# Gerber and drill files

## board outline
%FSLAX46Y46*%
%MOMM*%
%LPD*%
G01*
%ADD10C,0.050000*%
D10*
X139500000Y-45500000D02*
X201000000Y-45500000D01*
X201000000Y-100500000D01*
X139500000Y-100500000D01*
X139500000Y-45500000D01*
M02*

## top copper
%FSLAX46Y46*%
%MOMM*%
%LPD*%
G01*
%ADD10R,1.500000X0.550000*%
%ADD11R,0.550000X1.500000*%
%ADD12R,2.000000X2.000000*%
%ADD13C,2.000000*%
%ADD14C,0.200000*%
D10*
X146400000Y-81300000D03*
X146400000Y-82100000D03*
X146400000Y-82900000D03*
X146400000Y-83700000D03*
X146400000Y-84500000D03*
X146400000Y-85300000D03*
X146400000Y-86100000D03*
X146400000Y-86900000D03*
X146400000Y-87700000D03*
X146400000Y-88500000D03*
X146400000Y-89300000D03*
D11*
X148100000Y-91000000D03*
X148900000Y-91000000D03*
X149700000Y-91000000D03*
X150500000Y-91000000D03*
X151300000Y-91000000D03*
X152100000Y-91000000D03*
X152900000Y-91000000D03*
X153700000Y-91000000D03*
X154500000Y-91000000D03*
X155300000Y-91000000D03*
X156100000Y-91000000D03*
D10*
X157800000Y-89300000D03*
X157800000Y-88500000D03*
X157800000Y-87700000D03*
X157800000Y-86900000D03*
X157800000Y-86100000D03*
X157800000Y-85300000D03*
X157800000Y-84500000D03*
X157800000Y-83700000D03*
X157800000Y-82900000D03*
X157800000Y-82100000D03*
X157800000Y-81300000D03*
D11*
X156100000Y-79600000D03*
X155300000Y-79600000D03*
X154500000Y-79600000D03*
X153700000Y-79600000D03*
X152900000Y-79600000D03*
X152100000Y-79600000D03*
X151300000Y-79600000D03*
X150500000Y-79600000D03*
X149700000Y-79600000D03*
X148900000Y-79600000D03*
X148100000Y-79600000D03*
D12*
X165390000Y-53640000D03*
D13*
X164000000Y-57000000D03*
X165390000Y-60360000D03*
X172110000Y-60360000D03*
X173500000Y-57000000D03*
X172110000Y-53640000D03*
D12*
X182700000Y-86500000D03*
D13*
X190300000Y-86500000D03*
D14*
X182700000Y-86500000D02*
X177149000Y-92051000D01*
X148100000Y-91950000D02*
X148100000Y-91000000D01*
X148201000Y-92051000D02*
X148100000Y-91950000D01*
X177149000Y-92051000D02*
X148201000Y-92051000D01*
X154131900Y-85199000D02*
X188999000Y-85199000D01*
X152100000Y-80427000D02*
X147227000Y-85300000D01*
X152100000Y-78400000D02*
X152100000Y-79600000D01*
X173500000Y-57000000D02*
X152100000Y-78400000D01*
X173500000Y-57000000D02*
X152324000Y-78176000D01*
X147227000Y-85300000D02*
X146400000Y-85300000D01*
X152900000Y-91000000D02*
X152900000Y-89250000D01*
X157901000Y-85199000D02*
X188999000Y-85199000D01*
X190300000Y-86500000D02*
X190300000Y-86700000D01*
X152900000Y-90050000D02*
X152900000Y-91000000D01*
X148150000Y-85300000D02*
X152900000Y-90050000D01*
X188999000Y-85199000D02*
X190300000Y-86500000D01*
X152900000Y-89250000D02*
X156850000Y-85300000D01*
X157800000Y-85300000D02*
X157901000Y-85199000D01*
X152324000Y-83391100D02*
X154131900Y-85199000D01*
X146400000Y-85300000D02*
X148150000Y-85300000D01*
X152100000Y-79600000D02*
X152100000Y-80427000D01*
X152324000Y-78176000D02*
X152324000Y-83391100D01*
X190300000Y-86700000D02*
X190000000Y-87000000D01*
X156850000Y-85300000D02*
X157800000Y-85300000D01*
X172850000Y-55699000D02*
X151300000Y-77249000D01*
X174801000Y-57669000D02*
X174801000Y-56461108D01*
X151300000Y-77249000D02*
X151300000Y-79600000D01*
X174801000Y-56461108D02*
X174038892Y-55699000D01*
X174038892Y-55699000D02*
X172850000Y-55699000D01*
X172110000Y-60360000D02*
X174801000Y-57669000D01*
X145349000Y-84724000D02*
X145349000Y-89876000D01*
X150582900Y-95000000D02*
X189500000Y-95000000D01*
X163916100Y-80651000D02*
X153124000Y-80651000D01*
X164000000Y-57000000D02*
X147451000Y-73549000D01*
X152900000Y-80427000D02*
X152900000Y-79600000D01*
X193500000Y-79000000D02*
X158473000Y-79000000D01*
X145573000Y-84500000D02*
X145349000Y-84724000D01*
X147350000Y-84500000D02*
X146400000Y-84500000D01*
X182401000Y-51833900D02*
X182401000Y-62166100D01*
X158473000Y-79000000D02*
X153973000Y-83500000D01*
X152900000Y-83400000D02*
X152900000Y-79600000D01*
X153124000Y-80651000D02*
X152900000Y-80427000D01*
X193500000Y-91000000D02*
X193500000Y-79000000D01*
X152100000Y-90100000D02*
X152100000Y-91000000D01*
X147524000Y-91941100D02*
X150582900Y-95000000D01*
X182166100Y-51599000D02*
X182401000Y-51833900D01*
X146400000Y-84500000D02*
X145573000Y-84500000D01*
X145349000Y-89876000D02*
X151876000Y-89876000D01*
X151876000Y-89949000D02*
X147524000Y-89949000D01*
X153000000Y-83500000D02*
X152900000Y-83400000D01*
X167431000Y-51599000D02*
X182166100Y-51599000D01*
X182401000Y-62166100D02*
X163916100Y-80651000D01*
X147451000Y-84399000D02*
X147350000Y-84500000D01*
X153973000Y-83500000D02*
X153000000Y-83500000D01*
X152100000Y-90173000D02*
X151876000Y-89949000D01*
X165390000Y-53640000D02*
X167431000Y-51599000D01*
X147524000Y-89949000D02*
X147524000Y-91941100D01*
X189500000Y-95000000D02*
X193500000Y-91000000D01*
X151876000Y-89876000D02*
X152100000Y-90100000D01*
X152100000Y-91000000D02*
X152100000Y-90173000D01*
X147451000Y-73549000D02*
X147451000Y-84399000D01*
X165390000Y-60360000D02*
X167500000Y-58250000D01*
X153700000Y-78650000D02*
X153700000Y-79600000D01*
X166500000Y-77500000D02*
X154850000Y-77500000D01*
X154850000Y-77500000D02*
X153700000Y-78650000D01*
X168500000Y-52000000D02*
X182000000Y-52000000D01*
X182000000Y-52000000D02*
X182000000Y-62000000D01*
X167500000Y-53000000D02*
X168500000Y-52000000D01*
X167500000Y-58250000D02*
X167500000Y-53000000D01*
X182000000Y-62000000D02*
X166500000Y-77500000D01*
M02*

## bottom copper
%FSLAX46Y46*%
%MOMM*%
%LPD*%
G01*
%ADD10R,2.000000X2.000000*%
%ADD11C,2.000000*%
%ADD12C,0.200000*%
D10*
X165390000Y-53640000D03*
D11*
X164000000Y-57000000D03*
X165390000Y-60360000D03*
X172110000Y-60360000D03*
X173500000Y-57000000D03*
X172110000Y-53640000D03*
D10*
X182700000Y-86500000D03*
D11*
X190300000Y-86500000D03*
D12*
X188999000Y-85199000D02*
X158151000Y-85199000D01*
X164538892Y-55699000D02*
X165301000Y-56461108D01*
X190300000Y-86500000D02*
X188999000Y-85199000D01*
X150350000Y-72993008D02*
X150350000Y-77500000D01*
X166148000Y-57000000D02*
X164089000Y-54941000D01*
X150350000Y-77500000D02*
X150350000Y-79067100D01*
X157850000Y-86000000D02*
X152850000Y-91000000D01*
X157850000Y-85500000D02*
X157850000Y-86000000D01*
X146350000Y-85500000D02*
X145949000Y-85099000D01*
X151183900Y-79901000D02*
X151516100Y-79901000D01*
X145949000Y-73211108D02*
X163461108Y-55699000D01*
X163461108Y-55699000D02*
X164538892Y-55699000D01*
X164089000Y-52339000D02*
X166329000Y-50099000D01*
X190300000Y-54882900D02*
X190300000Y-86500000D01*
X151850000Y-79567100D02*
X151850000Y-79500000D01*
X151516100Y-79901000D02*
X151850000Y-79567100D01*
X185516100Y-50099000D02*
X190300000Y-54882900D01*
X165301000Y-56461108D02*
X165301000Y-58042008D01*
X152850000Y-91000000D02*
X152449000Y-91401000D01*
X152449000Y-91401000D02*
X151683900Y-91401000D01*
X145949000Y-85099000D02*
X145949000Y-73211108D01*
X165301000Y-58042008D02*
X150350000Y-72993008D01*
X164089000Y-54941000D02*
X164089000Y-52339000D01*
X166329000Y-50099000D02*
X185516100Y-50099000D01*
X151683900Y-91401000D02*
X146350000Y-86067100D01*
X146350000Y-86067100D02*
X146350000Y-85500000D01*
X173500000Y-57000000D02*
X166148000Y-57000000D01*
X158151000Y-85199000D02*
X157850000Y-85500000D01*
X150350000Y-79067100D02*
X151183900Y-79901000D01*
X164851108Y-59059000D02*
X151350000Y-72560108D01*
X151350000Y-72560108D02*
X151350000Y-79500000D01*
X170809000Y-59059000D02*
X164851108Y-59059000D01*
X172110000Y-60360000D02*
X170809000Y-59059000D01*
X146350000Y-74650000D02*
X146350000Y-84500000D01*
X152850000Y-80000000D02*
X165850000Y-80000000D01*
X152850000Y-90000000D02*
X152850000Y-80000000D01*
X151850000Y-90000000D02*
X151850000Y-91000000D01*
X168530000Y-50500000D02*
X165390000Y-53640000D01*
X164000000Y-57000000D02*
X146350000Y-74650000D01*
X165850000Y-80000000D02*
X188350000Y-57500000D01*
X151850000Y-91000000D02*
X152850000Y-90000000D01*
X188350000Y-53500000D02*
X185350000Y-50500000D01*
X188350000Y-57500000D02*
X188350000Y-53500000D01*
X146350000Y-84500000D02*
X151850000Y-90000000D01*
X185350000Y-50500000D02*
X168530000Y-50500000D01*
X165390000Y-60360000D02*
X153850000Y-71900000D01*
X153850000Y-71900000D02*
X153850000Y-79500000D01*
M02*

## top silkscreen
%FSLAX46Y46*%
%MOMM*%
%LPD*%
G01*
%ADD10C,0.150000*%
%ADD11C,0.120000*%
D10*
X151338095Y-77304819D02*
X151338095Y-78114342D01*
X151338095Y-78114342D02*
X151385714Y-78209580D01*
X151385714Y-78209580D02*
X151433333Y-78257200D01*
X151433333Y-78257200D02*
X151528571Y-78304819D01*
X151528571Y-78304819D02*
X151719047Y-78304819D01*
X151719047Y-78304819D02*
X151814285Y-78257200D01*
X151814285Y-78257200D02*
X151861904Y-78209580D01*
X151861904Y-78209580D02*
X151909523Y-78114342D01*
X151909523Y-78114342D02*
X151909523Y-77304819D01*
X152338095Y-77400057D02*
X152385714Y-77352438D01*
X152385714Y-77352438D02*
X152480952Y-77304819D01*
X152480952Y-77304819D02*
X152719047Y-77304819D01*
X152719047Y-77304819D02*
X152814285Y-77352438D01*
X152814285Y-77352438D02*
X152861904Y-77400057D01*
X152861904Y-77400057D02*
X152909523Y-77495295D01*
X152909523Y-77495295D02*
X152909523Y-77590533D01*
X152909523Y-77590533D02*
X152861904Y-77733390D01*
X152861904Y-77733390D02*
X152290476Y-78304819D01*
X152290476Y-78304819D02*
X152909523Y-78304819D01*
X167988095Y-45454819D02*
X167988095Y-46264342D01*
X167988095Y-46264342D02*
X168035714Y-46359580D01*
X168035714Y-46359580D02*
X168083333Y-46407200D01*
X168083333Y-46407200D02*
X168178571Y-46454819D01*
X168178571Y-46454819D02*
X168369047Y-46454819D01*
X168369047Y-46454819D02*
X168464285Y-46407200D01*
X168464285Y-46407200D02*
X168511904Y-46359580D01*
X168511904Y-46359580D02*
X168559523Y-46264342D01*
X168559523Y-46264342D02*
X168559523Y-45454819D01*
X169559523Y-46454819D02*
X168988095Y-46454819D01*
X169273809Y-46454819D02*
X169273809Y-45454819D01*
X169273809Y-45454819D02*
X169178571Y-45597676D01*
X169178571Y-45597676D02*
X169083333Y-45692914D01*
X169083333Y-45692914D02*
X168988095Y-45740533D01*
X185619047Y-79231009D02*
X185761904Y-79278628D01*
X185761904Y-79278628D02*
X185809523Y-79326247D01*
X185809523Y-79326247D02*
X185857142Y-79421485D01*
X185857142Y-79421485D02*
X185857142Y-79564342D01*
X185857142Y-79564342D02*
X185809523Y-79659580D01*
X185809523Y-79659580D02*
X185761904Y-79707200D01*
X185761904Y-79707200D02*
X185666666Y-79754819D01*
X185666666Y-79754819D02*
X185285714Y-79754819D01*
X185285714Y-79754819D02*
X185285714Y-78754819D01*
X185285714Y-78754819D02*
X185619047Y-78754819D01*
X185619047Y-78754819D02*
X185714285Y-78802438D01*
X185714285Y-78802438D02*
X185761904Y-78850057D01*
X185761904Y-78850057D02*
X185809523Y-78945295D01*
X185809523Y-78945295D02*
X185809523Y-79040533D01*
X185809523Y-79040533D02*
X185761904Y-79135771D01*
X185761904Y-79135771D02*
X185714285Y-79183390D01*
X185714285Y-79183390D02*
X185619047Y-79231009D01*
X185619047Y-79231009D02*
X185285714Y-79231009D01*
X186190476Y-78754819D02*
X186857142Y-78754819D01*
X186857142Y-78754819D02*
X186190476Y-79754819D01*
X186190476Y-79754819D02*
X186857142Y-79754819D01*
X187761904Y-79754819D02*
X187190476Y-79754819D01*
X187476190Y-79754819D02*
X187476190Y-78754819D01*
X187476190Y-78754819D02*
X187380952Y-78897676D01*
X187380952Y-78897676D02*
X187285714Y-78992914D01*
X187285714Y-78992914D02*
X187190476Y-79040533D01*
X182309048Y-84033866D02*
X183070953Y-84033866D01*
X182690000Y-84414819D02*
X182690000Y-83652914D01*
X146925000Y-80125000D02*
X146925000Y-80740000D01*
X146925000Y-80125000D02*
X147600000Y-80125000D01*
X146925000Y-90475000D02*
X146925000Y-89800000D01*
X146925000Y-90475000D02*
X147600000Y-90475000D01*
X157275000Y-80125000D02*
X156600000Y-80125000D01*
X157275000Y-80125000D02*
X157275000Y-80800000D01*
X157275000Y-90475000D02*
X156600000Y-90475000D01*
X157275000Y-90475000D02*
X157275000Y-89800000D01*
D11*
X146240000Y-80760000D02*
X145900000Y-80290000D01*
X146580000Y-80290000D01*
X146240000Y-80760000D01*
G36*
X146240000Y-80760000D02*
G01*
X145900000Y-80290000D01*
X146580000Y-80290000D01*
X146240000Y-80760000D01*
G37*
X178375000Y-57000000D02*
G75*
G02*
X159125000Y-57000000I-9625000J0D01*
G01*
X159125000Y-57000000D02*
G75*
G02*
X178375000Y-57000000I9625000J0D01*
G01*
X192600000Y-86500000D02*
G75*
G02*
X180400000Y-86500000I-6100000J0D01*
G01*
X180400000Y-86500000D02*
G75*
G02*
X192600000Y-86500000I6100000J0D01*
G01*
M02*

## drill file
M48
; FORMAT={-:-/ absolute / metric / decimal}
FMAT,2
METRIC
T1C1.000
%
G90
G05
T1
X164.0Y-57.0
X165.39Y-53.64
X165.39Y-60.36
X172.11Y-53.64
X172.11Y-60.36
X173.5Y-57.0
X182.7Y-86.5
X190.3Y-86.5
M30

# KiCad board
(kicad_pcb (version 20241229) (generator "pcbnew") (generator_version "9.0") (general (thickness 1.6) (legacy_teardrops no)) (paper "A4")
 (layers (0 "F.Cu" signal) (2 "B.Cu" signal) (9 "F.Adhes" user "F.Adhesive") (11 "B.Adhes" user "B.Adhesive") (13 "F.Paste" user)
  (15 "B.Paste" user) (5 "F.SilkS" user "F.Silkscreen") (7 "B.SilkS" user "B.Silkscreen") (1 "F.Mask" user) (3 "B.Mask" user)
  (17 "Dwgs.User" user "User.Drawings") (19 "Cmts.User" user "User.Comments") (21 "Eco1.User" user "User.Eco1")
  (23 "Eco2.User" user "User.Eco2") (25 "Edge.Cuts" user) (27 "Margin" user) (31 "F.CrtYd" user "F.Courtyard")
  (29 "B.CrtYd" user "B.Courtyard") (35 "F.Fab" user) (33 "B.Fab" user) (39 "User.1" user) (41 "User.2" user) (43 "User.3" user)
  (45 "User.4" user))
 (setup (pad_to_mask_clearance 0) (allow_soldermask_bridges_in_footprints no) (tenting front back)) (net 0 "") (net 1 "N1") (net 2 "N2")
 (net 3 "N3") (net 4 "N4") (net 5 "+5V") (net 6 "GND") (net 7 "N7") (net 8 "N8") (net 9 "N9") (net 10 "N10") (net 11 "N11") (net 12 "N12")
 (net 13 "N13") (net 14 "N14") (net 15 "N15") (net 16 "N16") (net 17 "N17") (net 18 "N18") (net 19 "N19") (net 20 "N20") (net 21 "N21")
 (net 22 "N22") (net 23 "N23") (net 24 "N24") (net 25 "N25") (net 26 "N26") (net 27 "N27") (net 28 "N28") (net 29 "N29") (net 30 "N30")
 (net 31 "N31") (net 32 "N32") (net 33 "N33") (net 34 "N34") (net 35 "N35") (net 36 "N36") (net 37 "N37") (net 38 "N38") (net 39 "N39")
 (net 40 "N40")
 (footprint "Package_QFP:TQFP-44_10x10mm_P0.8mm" (layer "F.Cu") (at 152.1 85.3)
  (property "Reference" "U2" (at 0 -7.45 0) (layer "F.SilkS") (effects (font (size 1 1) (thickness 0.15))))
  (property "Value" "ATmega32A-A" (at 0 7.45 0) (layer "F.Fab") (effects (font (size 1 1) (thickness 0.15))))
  (fp_line (start -5.175 -5.175) (end -5.175 -4.56) (stroke (width 0.15) (type solid)) (layer "F.SilkS"))
  (fp_line (start -5.175 -5.175) (end -4.5 -5.175) (stroke (width 0.15) (type solid)) (layer "F.SilkS"))
  (fp_line (start -5.175 5.175) (end -5.175 4.5) (stroke (width 0.15) (type solid)) (layer "F.SilkS"))
  (fp_line (start -5.175 5.175) (end -4.5 5.175) (stroke (width 0.15) (type solid)) (layer "F.SilkS"))
  (fp_line (start 5.175 -5.175) (end 4.5 -5.175) (stroke (width 0.15) (type solid)) (layer "F.SilkS"))
  (fp_line (start 5.175 -5.175) (end 5.175 -4.5) (stroke (width 0.15) (type solid)) (layer "F.SilkS"))
  (fp_line (start 5.175 5.175) (end 4.5 5.175) (stroke (width 0.15) (type solid)) (layer "F.SilkS"))
  (fp_line (start 5.175 5.175) (end 5.175 4.5) (stroke (width 0.15) (type solid)) (layer "F.SilkS"))
  (fp_poly
   (pts (xy -5.86 -4.54) (xy -6.2 -5.01) (xy -5.52 -5.01) (xy -5.86 -4.54)) (stroke (width 0.12) (type solid)) (fill yes) (layer "F.SilkS"))
  (pad "1" smd rect (at -5.7 -4) (size 1.5 0.55) (layers "F.Cu" "F.Mask" "F.Paste") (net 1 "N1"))
  (pad "2" smd rect (at -5.7 -3.2) (size 1.5 0.55) (layers "F.Cu" "F.Mask" "F.Paste") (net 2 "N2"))
  (pad "3" smd rect (at -5.7 -2.4) (size 1.5 0.55) (layers "F.Cu" "F.Mask" "F.Paste") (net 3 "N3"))
  (pad "4" smd rect (at -5.7 -1.6) (size 1.5 0.55) (layers "F.Cu" "F.Mask" "F.Paste") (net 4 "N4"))
  (pad "5" smd rect (at -5.7 -0.8) (size 1.5 0.55) (layers "F.Cu" "F.Mask" "F.Paste") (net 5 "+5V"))
  (pad "6" smd rect (at -5.7 0) (size 1.5 0.55) (layers "F.Cu" "F.Mask" "F.Paste") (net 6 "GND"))
  (pad "7" smd rect (at -5.7 0.8) (size 1.5 0.55) (layers "F.Cu" "F.Mask" "F.Paste") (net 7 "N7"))
  (pad "8" smd rect (at -5.7 1.6) (size 1.5 0.55) (layers "F.Cu" "F.Mask" "F.Paste") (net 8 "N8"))
  (pad "9" smd rect (at -5.7 2.4) (size 1.5 0.55) (layers "F.Cu" "F.Mask" "F.Paste") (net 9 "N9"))
  (pad "10" smd rect (at -5.7 3.2) (size 1.5 0.55) (layers "F.Cu" "F.Mask" "F.Paste") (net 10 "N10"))
  (pad "11" smd rect (at -5.7 4) (size 1.5 0.55) (layers "F.Cu" "F.Mask" "F.Paste") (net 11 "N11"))
  (pad "12" smd rect (at -4 5.7 90) (size 1.5 0.55) (layers "F.Cu" "F.Mask" "F.Paste") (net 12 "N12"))
  (pad "13" smd rect (at -3.2 5.7 90) (size 1.5 0.55) (layers "F.Cu" "F.Mask" "F.Paste") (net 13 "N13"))
  (pad "14" smd rect (at -2.4 5.7 90) (size 1.5 0.55) (layers "F.Cu" "F.Mask" "F.Paste") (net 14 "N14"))
  (pad "15" smd rect (at -1.6 5.7 90) (size 1.5 0.55) (layers "F.Cu" "F.Mask" "F.Paste") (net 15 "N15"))
  (pad "16" smd rect (at -0.8 5.7 90) (size 1.5 0.55) (layers "F.Cu" "F.Mask" "F.Paste") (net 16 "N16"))
  (pad "17" smd rect (at 0 5.7 90) (size 1.5 0.55) (layers "F.Cu" "F.Mask" "F.Paste") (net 5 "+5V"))
  (pad "18" smd rect (at 0.8 5.7 90) (size 1.5 0.55) (layers "F.Cu" "F.Mask" "F.Paste") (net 6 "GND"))
  (pad "19" smd rect (at 1.6 5.7 90) (size 1.5 0.55) (layers "F.Cu" "F.Mask" "F.Paste") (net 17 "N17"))
  (pad "20" smd rect (at 2.4 5.7 90) (size 1.5 0.55) (layers "F.Cu" "F.Mask" "F.Paste") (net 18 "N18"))
  (pad "21" smd rect (at 3.2 5.7 90) (size 1.5 0.55) (layers "F.Cu" "F.Mask" "F.Paste") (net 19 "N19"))
  (pad "22" smd rect (at 4 5.7 90) (size 1.5 0.55) (layers "F.Cu" "F.Mask" "F.Paste") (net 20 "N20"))
  (pad "23" smd rect (at 5.7 4) (size 1.5 0.55) (layers "F.Cu" "F.Mask" "F.Paste") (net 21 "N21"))
  (pad "24" smd rect (at 5.7 3.2) (size 1.5 0.55) (layers "F.Cu" "F.Mask" "F.Paste") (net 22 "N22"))
  (pad "25" smd rect (at 5.7 2.4) (size 1.5 0.55) (layers "F.Cu" "F.Mask" "F.Paste") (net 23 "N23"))
  (pad "26" smd rect (at 5.7 1.6) (size 1.5 0.55) (layers "F.Cu" "F.Mask" "F.Paste") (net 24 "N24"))
  (pad "27" smd rect (at 5.7 0.8) (size 1.5 0.55) (layers "F.Cu" "F.Mask" "F.Paste") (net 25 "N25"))
  (pad "28" smd rect (at 5.7 0) (size 1.5 0.55) (layers "F.Cu" "F.Mask" "F.Paste") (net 6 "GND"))
  (pad "29" smd rect (at 5.7 -0.8) (size 1.5 0.55) (layers "F.Cu" "F.Mask" "F.Paste") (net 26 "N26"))
  (pad "30" smd rect (at 5.7 -1.6) (size 1.5 0.55) (layers "F.Cu" "F.Mask" "F.Paste") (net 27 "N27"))
  (pad "31" smd rect (at 5.7 -2.4) (size 1.5 0.55) (layers "F.Cu" "F.Mask" "F.Paste") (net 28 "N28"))
  (pad "32" smd rect (at 5.7 -3.2) (size 1.5 0.55) (layers "F.Cu" "F.Mask" "F.Paste") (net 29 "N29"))
  (pad "33" smd rect (at 5.7 -4) (size 1.5 0.55) (layers "F.Cu" "F.Mask" "F.Paste") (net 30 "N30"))
  (pad "34" smd rect (at 4 -5.7 90) (size 1.5 0.55) (layers "F.Cu" "F.Mask" "F.Paste") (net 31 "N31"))
  (pad "35" smd rect (at 3.2 -5.7 90) (size 1.5 0.55) (layers "F.Cu" "F.Mask" "F.Paste") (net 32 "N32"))
  (pad "36" smd rect (at 2.4 -5.7 90) (size 1.5 0.55) (layers "F.Cu" "F.Mask" "F.Paste") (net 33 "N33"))
  (pad "37" smd rect (at 1.6 -5.7 90) (size 1.5 0.55) (layers "F.Cu" "F.Mask" "F.Paste") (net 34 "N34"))
  (pad "38" smd rect (at 0.8 -5.7 90) (size 1.5 0.55) (layers "F.Cu" "F.Mask" "F.Paste") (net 5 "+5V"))
  (pad "39" smd rect (at 0 -5.7 90) (size 1.5 0.55) (layers "F.Cu" "F.Mask" "F.Paste") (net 6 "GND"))
  (pad "40" smd rect (at -0.8 -5.7 90) (size 1.5 0.55) (layers "F.Cu" "F.Mask" "F.Paste") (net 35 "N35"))
  (pad "41" smd rect (at -1.6 -5.7 90) (size 1.5 0.55) (layers "F.Cu" "F.Mask" "F.Paste") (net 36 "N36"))
  (pad "42" smd rect (at -2.4 -5.7 90) (size 1.5 0.55) (layers "F.Cu" "F.Mask" "F.Paste") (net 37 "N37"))
  (pad "43" smd rect (at -3.2 -5.7 90) (size 1.5 0.55) (layers "F.Cu" "F.Mask" "F.Paste") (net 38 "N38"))
  (pad "44" smd rect (at -4 -5.7 90) (size 1.5 0.55) (layers "F.Cu" "F.Mask" "F.Paste") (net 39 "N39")))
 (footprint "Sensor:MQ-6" (layer "F.Cu") (at 165.39 53.64)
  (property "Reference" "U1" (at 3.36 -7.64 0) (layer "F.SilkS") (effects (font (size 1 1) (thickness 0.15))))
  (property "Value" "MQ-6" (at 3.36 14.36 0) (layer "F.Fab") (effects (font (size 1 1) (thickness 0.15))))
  (fp_circle (center 3.36 3.36) (end 12.985 3.36) (stroke (width 0.12) (type solid)) (fill no) (layer "F.SilkS"))
  (pad "1" thru_hole rect (at 0 0) (size 2 2) (drill 1) (layers "*.Cu" "*.Mask") (remove_unused_layers no) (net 5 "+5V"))
  (pad "2" thru_hole circle (at -1.39 3.36) (size 2 2) (drill 1) (layers "*.Cu" "*.Mask") (remove_unused_layers no) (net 5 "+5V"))
  (pad "3" thru_hole circle (at 0 6.72 90) (size 2 2) (drill 1) (layers "*.Cu" "*.Mask") (remove_unused_layers no) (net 34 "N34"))
  (pad "4" thru_hole circle (at 6.72 6.72 180) (size 2 2) (drill 1) (layers "*.Cu" "*.Mask") (remove_unused_layers no) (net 35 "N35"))
  (pad "5" thru_hole circle (at 8.11 3.36) (size 2 2) (drill 1) (layers "*.Cu" "*.Mask") (remove_unused_layers no) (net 6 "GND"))
  (pad "6" thru_hole circle (at 6.72 0 270) (size 2 2) (drill 1) (layers "*.Cu" "*.Mask") (remove_unused_layers no) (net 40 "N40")))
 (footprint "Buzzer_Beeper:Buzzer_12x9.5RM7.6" (layer "F.Cu") (at 182.7 86.5)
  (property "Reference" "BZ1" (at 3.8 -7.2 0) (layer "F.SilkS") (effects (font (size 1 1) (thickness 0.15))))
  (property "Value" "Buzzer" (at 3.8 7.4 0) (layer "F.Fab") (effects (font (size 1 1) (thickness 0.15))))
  (fp_circle (center 3.8 0) (end 9.9 0) (stroke (width 0.12) (type solid)) (fill no) (layer "F.SilkS"))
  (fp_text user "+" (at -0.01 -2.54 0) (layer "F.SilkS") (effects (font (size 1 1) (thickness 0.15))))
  (pad "1" thru_hole rect (at 0 0) (size 2 2) (drill 1) (layers "*.Cu" "*.Mask") (remove_unused_layers no) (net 12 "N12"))
  (pad "2" thru_hole circle (at 7.6 0) (size 2 2) (drill 1) (layers "*.Cu" "*.Mask") (remove_unused_layers no) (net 6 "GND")))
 (gr_rect (start 139.5 45.5) (end 201 100.5) (stroke (width 0.05) (type default)) (fill no) (layer "Edge.Cuts"))
 (segment (start 182.7 86.5) (end 177.149 92.051) (width 0.2) (layer "F.Cu") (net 12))
 (segment (start 148.1 91.95) (end 148.1 91) (width 0.2) (layer "F.Cu") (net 12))
 (segment (start 148.201 92.051) (end 148.1 91.95) (width 0.2) (layer "F.Cu") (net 12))
 (segment (start 177.149 92.051) (end 148.201 92.051) (width 0.2) (layer "F.Cu") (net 12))
 (segment (start 154.1319 85.199) (end 188.999 85.199) (width 0.2) (layer "F.Cu") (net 6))
 (segment (start 152.1 80.427) (end 147.227 85.3) (width 0.2) (layer "F.Cu") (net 6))
 (segment (start 152.1 78.4) (end 152.1 79.6) (width 0.2) (layer "F.Cu") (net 6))
 (segment (start 173.5 57) (end 152.1 78.4) (width 0.2) (layer "F.Cu") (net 6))
 (segment (start 173.5 57) (end 152.324 78.176) (width 0.2) (layer "F.Cu") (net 6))
 (segment (start 147.227 85.3) (end 146.4 85.3) (width 0.2) (layer "F.Cu") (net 6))
 (segment (start 152.9 91) (end 152.9 89.25) (width 0.2) (layer "F.Cu") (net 6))
 (segment (start 157.901 85.199) (end 188.999 85.199) (width 0.2) (layer "F.Cu") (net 6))
 (segment (start 190.3 86.5) (end 190.3 86.7) (width 0.2) (layer "F.Cu") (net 6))
 (segment (start 152.9 90.05) (end 152.9 91) (width 0.2) (layer "F.Cu") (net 6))
 (segment (start 148.15 85.3) (end 152.9 90.05) (width 0.2) (layer "F.Cu") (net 6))
 (segment (start 188.999 85.199) (end 190.3 86.5) (width 0.2) (layer "F.Cu") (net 6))
 (segment (start 152.9 89.25) (end 156.85 85.3) (width 0.2) (layer "F.Cu") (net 6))
 (segment (start 157.8 85.3) (end 157.901 85.199) (width 0.2) (layer "F.Cu") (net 6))
 (segment (start 152.324 83.3911) (end 154.1319 85.199) (width 0.2) (layer "F.Cu") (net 6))
 (segment (start 146.4 85.3) (end 148.15 85.3) (width 0.2) (layer "F.Cu") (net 6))
 (segment (start 152.1 79.6) (end 152.1 80.427) (width 0.2) (layer "F.Cu") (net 6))
 (segment (start 152.324 78.176) (end 152.324 83.3911) (width 0.2) (layer "F.Cu") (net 6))
 (segment (start 190.3 86.7) (end 190 87) (width 0.2) (layer "F.Cu") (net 6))
 (segment (start 156.85 85.3) (end 157.8 85.3) (width 0.2) (layer "F.Cu") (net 6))
 (segment (start 188.999 85.199) (end 158.151 85.199) (width 0.2) (layer "B.Cu") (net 6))
 (segment (start 164.538892 55.699) (end 165.301 56.461108) (width 0.2) (layer "B.Cu") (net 6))
 (segment (start 190.3 86.5) (end 188.999 85.199) (width 0.2) (layer "B.Cu") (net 6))
 (segment (start 150.35 72.993008) (end 150.35 77.5) (width 0.2) (layer "B.Cu") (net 6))
 (segment (start 166.148 57) (end 164.089 54.941) (width 0.2) (layer "B.Cu") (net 6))
 (segment (start 150.35 77.5) (end 150.35 79.0671) (width 0.2) (layer "B.Cu") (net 6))
 (segment (start 157.85 86) (end 152.85 91) (width 0.2) (layer "B.Cu") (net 6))
 (segment (start 157.85 85.5) (end 157.85 86) (width 0.2) (layer "B.Cu") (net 6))
 (segment (start 146.35 85.5) (end 145.949 85.099) (width 0.2) (layer "B.Cu") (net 6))
 (segment (start 151.1839 79.901) (end 151.5161 79.901) (width 0.2) (layer "B.Cu") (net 6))
 (segment (start 145.949 73.211108) (end 163.461108 55.699) (width 0.2) (layer "B.Cu") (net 6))
 (segment (start 163.461108 55.699) (end 164.538892 55.699) (width 0.2) (layer "B.Cu") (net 6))
 (segment (start 164.089 52.339) (end 166.329 50.099) (width 0.2) (layer "B.Cu") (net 6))
 (segment (start 190.3 54.8829) (end 190.3 86.5) (width 0.2) (layer "B.Cu") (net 6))
 (segment (start 151.85 79.5671) (end 151.85 79.5) (width 0.2) (layer "B.Cu") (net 6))
 (segment (start 151.5161 79.901) (end 151.85 79.5671) (width 0.2) (layer "B.Cu") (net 6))
 (segment (start 185.5161 50.099) (end 190.3 54.8829) (width 0.2) (layer "B.Cu") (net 6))
 (segment (start 165.301 56.461108) (end 165.301 58.042008) (width 0.2) (layer "B.Cu") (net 6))
 (segment (start 152.85 91) (end 152.449 91.401) (width 0.2) (layer "B.Cu") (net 6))
 (segment (start 152.449 91.401) (end 151.6839 91.401) (width 0.2) (layer "B.Cu") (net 6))
 (segment (start 145.949 85.099) (end 145.949 73.211108) (width 0.2) (layer "B.Cu") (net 6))
 (segment (start 165.301 58.042008) (end 150.35 72.993008) (width 0.2) (layer "B.Cu") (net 6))
 (segment (start 164.089 54.941) (end 164.089 52.339) (width 0.2) (layer "B.Cu") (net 6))
 (segment (start 166.329 50.099) (end 185.5161 50.099) (width 0.2) (layer "B.Cu") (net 6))
 (segment (start 151.6839 91.401) (end 146.35 86.0671) (width 0.2) (layer "B.Cu") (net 6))
 (segment (start 146.35 86.0671) (end 146.35 85.5) (width 0.2) (layer "B.Cu") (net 6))
 (segment (start 173.5 57) (end 166.148 57) (width 0.2) (layer "B.Cu") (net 6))
 (segment (start 158.151 85.199) (end 157.85 85.5) (width 0.2) (layer "B.Cu") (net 6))
 (segment (start 150.35 79.0671) (end 151.1839 79.901) (width 0.2) (layer "B.Cu") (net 6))
 (segment (start 172.85 55.699) (end 151.3 77.249) (width 0.2) (layer "F.Cu") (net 35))
 (segment (start 174.801 57.669) (end 174.801 56.461108) (width 0.2) (layer "F.Cu") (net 35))
 (segment (start 151.3 77.249) (end 151.3 79.6) (width 0.2) (layer "F.Cu") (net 35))
 (segment (start 174.801 56.461108) (end 174.038892 55.699) (width 0.2) (layer "F.Cu") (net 35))
 (segment (start 174.038892 55.699) (end 172.85 55.699) (width 0.2) (layer "F.Cu") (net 35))
 (segment (start 172.11 60.36) (end 174.801 57.669) (width 0.2) (layer "F.Cu") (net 35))
 (segment (start 164.851108 59.059) (end 151.35 72.560108) (width 0.2) (layer "B.Cu") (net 35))
 (segment (start 151.35 72.560108) (end 151.35 79.5) (width 0.2) (layer "B.Cu") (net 35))
 (segment (start 170.809 59.059) (end 164.851108 59.059) (width 0.2) (layer "B.Cu") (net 35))
 (segment (start 172.11 60.36) (end 170.809 59.059) (width 0.2) (layer "B.Cu") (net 35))
 (segment (start 145.349 84.724) (end 145.349 89.876) (width 0.2) (layer "F.Cu") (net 5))
 (segment (start 150.5829 95) (end 189.5 95) (width 0.2) (layer "F.Cu") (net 5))
 (segment (start 163.9161 80.651) (end 153.124 80.651) (width 0.2) (layer "F.Cu") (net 5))
 (segment (start 164 57) (end 147.451 73.549) (width 0.2) (layer "F.Cu") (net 5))
 (segment (start 152.9 80.427) (end 152.9 79.6) (width 0.2) (layer "F.Cu") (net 5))
 (segment (start 193.5 79) (end 158.473 79) (width 0.2) (layer "F.Cu") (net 5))
 (segment (start 145.573 84.5) (end 145.349 84.724) (width 0.2) (layer "F.Cu") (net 5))
 (segment (start 147.35 84.5) (end 146.4 84.5) (width 0.2) (layer "F.Cu") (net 5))
 (segment (start 182.401 51.8339) (end 182.401 62.1661) (width 0.2) (layer "F.Cu") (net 5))
 (segment (start 158.473 79) (end 153.973 83.5) (width 0.2) (layer "F.Cu") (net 5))
 (segment (start 152.9 83.4) (end 152.9 79.6) (width 0.2) (layer "F.Cu") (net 5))
 (segment (start 153.124 80.651) (end 152.9 80.427) (width 0.2) (layer "F.Cu") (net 5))
 (segment (start 193.5 91) (end 193.5 79) (width 0.2) (layer "F.Cu") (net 5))
 (segment (start 152.1 90.1) (end 152.1 91) (width 0.2) (layer "F.Cu") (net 5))
 (segment (start 147.524 91.9411) (end 150.5829 95) (width 0.2) (layer "F.Cu") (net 5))
 (segment (start 182.1661 51.599) (end 182.401 51.8339) (width 0.2) (layer "F.Cu") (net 5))
 (segment (start 146.4 84.5) (end 145.573 84.5) (width 0.2) (layer "F.Cu") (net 5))
 (segment (start 145.349 89.876) (end 151.876 89.876) (width 0.2) (layer "F.Cu") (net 5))
 (segment (start 151.876 89.949) (end 147.524 89.949) (width 0.2) (layer "F.Cu") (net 5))
 (segment (start 153 83.5) (end 152.9 83.4) (width 0.2) (layer "F.Cu") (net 5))
 (segment (start 167.431 51.599) (end 182.1661 51.599) (width 0.2) (layer "F.Cu") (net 5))
 (segment (start 182.401 62.1661) (end 163.9161 80.651) (width 0.2) (layer "F.Cu") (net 5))
 (segment (start 147.451 84.399) (end 147.35 84.5) (width 0.2) (layer "F.Cu") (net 5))
 (segment (start 153.973 83.5) (end 153 83.5) (width 0.2) (layer "F.Cu") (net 5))
 (segment (start 152.1 90.173) (end 151.876 89.949) (width 0.2) (layer "F.Cu") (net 5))
 (segment (start 165.39 53.64) (end 167.431 51.599) (width 0.2) (layer "F.Cu") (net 5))
 (segment (start 147.524 89.949) (end 147.524 91.9411) (width 0.2) (layer "F.Cu") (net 5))
 (segment (start 189.5 95) (end 193.5 91) (width 0.2) (layer "F.Cu") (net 5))
 (segment (start 151.876 89.876) (end 152.1 90.1) (width 0.2) (layer "F.Cu") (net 5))
 (segment (start 152.1 91) (end 152.1 90.173) (width 0.2) (layer "F.Cu") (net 5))
 (segment (start 147.451 73.549) (end 147.451 84.399) (width 0.2) (layer "F.Cu") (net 5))
 (segment (start 146.35 74.65) (end 146.35 84.5) (width 0.2) (layer "B.Cu") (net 5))
 (segment (start 152.85 80) (end 165.85 80) (width 0.2) (layer "B.Cu") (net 5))
 (segment (start 152.85 90) (end 152.85 80) (width 0.2) (layer "B.Cu") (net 5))
 (segment (start 151.85 90) (end 151.85 91) (width 0.2) (layer "B.Cu") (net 5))
 (segment (start 168.53 50.5) (end 165.39 53.64) (width 0.2) (layer "B.Cu") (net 5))
 (segment (start 164 57) (end 146.35 74.65) (width 0.2) (layer "B.Cu") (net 5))
 (segment (start 165.85 80) (end 188.35 57.5) (width 0.2) (layer "B.Cu") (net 5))
 (segment (start 151.85 91) (end 152.85 90) (width 0.2) (layer "B.Cu") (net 5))
 (segment (start 188.35 53.5) (end 185.35 50.5) (width 0.2) (layer "B.Cu") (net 5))
 (segment (start 188.35 57.5) (end 188.35 53.5) (width 0.2) (layer "B.Cu") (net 5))
 (segment (start 146.35 84.5) (end 151.85 90) (width 0.2) (layer "B.Cu") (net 5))
 (segment (start 185.35 50.5) (end 168.53 50.5) (width 0.2) (layer "B.Cu") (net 5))
 (segment (start 165.39 60.36) (end 167.5 58.25) (width 0.2) (layer "F.Cu") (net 34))
 (segment (start 153.7 78.65) (end 153.7 79.6) (width 0.2) (layer "F.Cu") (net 34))
 (segment (start 166.5 77.5) (end 154.85 77.5) (width 0.2) (layer "F.Cu") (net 34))
 (segment (start 154.85 77.5) (end 153.7 78.65) (width 0.2) (layer "F.Cu") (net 34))
 (segment (start 168.5 52) (end 182 52) (width 0.2) (layer "F.Cu") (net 34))
 (segment (start 182 52) (end 182 62) (width 0.2) (layer "F.Cu") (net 34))
 (segment (start 167.5 53) (end 168.5 52) (width 0.2) (layer "F.Cu") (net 34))
 (segment (start 167.5 58.25) (end 167.5 53) (width 0.2) (layer "F.Cu") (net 34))
 (segment (start 182 62) (end 166.5 77.5) (width 0.2) (layer "F.Cu") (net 34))
 (segment (start 165.39 60.36) (end 153.85 71.9) (width 0.2) (layer "B.Cu") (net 34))
 (segment (start 153.85 71.9) (end 153.85 79.5) (width 0.2) (layer "B.Cu") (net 34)))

